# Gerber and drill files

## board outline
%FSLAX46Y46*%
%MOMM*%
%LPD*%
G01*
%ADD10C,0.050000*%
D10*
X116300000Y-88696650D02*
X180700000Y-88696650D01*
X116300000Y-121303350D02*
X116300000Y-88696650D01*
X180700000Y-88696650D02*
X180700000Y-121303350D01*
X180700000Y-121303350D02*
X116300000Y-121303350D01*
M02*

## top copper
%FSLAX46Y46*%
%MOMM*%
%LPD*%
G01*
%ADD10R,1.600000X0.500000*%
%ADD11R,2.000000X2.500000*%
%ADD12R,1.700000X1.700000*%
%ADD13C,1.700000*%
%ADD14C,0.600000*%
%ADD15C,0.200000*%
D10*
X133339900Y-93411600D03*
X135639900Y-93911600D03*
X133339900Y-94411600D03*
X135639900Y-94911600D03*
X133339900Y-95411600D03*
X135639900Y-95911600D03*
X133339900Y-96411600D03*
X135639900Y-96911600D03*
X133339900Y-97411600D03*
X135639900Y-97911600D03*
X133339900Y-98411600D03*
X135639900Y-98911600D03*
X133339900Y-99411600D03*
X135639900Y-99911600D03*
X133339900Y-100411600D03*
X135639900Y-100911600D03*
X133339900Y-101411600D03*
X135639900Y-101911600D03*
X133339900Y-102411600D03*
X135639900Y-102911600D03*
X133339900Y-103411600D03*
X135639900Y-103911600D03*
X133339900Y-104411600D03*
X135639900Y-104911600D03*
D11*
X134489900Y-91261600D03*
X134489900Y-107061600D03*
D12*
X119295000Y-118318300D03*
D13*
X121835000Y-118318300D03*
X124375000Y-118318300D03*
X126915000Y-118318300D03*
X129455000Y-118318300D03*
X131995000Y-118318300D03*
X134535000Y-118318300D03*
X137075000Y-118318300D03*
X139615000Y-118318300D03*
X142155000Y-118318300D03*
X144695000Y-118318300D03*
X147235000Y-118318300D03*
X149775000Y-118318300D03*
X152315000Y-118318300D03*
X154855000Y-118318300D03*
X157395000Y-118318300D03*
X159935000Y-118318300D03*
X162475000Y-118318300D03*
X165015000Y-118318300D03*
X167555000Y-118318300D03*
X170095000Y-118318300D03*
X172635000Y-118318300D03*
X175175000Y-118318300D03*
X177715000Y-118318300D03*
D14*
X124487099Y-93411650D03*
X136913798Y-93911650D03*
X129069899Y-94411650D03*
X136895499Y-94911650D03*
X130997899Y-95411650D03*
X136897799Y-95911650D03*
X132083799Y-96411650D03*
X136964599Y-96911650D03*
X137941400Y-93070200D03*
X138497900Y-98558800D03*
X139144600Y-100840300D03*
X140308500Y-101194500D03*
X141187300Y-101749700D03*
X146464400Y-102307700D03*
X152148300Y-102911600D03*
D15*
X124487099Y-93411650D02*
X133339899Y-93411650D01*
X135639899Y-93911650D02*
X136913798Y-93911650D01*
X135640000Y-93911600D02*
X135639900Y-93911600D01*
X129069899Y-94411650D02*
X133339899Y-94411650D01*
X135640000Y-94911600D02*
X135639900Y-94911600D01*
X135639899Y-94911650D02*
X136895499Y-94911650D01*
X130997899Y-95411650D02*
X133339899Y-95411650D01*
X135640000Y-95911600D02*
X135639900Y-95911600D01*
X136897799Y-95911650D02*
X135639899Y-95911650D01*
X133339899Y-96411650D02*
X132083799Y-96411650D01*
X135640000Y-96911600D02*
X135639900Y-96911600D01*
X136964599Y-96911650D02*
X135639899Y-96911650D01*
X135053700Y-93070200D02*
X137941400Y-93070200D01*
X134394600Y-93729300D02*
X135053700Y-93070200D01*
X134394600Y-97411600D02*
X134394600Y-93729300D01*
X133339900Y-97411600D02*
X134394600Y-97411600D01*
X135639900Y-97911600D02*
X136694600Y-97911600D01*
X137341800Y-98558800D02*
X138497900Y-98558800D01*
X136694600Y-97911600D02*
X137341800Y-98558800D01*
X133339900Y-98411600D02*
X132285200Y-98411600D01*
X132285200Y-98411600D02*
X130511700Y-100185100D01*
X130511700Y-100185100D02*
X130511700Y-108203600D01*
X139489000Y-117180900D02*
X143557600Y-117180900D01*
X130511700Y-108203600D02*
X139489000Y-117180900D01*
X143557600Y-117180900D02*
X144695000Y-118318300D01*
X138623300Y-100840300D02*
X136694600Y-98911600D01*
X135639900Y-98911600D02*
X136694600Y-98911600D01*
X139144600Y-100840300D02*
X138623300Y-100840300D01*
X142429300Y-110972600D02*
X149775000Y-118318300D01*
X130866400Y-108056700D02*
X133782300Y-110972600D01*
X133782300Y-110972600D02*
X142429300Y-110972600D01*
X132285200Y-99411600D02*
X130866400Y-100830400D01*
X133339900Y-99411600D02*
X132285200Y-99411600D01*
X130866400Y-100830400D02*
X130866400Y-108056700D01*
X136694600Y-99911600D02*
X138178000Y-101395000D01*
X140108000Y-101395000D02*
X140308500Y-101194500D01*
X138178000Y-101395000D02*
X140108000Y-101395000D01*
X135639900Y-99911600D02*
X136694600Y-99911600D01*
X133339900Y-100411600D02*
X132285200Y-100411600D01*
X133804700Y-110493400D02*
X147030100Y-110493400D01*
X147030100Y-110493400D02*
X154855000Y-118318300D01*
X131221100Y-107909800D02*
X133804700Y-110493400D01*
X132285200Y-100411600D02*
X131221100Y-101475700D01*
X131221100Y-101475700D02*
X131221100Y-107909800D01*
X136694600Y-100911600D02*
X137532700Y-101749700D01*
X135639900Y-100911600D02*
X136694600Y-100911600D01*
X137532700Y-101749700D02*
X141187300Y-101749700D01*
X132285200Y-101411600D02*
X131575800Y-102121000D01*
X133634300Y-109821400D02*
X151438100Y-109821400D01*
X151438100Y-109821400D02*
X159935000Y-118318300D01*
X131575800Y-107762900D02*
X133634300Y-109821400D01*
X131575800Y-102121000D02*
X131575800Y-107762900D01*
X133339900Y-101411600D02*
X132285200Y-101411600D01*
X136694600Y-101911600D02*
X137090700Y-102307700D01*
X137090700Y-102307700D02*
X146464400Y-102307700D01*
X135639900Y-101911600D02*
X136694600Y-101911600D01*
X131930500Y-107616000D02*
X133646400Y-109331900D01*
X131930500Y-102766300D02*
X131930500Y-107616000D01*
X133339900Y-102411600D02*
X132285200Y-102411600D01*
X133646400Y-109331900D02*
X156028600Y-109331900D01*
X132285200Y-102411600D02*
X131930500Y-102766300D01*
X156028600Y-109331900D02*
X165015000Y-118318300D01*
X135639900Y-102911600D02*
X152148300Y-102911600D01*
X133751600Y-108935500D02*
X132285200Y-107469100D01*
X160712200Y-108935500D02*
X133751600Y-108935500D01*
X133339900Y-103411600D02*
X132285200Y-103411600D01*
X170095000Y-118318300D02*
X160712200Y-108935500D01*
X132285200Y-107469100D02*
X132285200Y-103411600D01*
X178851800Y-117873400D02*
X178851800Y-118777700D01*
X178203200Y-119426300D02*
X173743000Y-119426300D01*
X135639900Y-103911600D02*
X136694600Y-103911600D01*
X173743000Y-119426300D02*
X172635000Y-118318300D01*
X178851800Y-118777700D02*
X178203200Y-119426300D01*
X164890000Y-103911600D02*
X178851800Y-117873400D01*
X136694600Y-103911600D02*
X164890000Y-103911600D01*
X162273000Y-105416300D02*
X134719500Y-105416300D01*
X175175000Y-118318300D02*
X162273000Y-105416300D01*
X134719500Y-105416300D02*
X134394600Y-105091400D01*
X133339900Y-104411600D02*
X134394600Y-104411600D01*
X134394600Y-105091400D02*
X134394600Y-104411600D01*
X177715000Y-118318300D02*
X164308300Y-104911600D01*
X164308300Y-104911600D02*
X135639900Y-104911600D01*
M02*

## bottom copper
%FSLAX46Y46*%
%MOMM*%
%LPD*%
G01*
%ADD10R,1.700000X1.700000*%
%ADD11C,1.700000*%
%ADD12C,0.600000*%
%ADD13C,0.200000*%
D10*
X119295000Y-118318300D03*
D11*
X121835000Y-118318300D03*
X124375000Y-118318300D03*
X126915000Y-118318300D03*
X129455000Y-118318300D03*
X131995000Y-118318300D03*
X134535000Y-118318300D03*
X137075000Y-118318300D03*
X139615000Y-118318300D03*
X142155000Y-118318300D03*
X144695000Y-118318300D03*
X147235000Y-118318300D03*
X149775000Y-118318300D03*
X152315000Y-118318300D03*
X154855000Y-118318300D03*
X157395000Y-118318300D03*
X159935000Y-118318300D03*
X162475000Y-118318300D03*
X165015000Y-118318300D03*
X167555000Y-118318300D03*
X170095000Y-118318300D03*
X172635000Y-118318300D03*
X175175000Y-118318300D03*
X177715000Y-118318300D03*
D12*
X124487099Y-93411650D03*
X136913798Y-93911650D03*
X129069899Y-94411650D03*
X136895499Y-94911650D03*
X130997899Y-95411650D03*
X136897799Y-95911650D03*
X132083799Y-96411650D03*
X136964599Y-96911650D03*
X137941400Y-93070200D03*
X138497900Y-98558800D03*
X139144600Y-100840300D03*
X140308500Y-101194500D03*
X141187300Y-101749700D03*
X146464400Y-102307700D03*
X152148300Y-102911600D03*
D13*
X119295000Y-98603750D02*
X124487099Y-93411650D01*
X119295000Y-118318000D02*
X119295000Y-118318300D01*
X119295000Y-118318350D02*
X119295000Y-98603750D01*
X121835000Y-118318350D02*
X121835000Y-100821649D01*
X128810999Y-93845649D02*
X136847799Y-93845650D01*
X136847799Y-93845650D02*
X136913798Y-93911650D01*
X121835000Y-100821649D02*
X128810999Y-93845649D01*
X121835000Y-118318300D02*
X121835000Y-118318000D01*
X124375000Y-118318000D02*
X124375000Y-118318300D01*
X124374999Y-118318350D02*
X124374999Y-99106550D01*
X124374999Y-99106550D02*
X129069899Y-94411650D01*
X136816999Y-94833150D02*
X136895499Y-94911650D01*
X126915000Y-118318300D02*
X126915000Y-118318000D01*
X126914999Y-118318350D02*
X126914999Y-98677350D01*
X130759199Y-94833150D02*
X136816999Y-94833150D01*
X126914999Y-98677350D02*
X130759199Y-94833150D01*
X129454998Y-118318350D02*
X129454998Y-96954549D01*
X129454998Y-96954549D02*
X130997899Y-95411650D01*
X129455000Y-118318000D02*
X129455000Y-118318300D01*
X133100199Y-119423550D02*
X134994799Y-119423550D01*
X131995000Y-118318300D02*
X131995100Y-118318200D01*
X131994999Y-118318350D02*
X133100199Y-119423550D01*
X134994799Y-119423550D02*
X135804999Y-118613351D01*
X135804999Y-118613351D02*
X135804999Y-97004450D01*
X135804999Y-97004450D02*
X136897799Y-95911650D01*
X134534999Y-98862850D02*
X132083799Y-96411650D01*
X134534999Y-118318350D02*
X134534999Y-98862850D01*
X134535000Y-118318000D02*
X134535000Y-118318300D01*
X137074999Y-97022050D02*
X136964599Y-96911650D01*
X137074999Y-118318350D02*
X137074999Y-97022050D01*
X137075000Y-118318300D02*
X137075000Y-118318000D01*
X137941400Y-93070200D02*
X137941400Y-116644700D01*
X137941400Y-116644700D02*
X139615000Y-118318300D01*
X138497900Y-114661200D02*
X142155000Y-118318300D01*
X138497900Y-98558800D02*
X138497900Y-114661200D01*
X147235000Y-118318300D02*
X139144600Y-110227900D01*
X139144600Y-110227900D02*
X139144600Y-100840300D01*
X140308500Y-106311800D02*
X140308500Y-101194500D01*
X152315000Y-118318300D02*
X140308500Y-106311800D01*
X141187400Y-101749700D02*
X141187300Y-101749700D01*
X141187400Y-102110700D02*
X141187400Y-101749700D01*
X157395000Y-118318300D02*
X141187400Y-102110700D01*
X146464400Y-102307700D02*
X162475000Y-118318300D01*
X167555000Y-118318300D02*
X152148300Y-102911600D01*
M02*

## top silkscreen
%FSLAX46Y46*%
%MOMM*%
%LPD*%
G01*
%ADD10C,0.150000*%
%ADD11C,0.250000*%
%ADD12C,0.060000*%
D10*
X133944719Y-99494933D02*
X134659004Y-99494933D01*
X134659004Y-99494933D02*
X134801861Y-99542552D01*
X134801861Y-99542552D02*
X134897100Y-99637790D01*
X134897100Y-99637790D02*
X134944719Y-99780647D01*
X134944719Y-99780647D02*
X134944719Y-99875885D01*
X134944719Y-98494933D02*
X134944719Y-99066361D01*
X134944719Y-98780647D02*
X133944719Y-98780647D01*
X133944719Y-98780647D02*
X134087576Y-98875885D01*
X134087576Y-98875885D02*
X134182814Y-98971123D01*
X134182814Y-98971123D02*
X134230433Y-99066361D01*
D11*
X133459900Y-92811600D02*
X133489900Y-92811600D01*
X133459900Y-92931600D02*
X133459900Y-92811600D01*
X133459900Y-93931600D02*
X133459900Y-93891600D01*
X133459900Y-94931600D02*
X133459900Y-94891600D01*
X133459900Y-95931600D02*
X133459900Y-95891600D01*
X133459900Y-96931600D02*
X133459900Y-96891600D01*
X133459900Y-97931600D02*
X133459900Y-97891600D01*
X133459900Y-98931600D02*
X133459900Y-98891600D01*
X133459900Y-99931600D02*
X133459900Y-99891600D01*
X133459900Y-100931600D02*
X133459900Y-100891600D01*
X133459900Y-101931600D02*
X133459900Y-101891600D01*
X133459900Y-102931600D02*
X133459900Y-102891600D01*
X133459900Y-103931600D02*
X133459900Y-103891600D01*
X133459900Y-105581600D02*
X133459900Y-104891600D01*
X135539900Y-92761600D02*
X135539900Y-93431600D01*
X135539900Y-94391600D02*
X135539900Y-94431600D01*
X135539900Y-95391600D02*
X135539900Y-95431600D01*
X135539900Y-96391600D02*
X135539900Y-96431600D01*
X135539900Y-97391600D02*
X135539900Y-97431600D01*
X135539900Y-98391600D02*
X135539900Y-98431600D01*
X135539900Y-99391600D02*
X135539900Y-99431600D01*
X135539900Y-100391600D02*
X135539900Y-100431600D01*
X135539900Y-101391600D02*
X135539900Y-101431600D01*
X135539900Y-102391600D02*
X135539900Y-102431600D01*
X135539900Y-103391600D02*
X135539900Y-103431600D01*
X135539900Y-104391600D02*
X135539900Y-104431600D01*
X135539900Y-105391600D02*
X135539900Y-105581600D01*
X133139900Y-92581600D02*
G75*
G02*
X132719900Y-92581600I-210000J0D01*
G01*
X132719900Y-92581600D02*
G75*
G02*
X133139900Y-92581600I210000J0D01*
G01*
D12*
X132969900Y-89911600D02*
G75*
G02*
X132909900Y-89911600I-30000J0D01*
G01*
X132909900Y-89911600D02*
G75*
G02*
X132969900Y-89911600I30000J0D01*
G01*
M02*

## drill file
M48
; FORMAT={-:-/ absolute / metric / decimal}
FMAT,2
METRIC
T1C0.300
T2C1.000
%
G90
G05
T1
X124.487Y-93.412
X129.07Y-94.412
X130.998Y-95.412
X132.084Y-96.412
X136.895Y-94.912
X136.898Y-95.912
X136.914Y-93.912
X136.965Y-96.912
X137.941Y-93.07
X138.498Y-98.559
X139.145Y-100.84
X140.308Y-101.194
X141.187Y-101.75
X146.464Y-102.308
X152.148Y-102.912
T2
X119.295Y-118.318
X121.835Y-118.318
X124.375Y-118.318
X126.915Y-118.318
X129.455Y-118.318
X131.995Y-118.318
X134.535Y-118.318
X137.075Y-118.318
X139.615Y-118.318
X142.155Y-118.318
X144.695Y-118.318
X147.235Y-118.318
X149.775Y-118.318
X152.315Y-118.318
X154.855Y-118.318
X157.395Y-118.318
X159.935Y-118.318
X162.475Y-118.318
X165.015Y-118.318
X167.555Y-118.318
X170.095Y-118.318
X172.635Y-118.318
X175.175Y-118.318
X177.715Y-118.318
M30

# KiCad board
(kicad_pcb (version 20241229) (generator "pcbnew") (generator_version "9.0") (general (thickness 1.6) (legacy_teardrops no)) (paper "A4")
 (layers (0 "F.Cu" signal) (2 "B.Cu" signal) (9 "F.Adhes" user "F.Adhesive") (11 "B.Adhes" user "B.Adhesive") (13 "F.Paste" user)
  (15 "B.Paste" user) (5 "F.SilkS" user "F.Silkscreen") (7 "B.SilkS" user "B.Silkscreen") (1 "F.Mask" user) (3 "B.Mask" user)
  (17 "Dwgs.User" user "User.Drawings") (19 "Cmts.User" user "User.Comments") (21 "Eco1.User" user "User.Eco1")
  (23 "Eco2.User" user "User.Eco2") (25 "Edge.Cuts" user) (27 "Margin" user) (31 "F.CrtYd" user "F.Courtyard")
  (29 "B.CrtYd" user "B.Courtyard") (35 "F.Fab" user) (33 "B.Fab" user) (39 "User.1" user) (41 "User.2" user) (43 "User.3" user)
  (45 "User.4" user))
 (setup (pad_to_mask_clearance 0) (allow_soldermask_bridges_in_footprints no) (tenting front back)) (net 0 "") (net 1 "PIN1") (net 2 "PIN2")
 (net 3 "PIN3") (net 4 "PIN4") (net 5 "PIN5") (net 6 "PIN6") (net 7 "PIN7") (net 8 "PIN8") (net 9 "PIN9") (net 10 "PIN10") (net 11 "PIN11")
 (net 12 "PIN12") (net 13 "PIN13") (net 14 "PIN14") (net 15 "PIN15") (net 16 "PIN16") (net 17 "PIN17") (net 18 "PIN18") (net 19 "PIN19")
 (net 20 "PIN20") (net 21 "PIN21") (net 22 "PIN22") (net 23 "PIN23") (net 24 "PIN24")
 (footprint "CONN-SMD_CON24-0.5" (layer "F.Cu") (at 134.4899 99.1616 -90)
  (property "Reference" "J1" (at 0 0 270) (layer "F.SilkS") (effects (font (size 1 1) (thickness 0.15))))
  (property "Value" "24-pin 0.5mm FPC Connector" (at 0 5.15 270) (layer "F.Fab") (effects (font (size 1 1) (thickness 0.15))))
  (fp_line (start -6.35 1.03) (end -6.35 1) (stroke (width 0.25) (type solid)) (layer "F.SilkS"))
  (fp_line (start -6.23 1.03) (end -6.35 1.03) (stroke (width 0.25) (type solid)) (layer "F.SilkS"))
  (fp_line (start -5.23 1.03) (end -5.27 1.03) (stroke (width 0.25) (type solid)) (layer "F.SilkS"))
  (fp_line (start -4.23 1.03) (end -4.27 1.03) (stroke (width 0.25) (type solid)) (layer "F.SilkS"))
  (fp_line (start -3.23 1.03) (end -3.27 1.03) (stroke (width 0.25) (type solid)) (layer "F.SilkS"))
  (fp_line (start -2.23 1.03) (end -2.27 1.03) (stroke (width 0.25) (type solid)) (layer "F.SilkS"))
  (fp_line (start -1.23 1.03) (end -1.27 1.03) (stroke (width 0.25) (type solid)) (layer "F.SilkS"))
  (fp_line (start -0.23 1.03) (end -0.27 1.03) (stroke (width 0.25) (type solid)) (layer "F.SilkS"))
  (fp_line (start 0.77 1.03) (end 0.73 1.03) (stroke (width 0.25) (type solid)) (layer "F.SilkS"))
  (fp_line (start 1.77 1.03) (end 1.73 1.03) (stroke (width 0.25) (type solid)) (layer "F.SilkS"))
  (fp_line (start 2.77 1.03) (end 2.73 1.03) (stroke (width 0.25) (type solid)) (layer "F.SilkS"))
  (fp_line (start 3.77 1.03) (end 3.73 1.03) (stroke (width 0.25) (type solid)) (layer "F.SilkS"))
  (fp_line (start 4.77 1.03) (end 4.73 1.03) (stroke (width 0.25) (type solid)) (layer "F.SilkS"))
  (fp_line (start 6.42 1.03) (end 5.73 1.03) (stroke (width 0.25) (type solid)) (layer "F.SilkS"))
  (fp_line (start -6.4 -1.05) (end -5.73 -1.05) (stroke (width 0.25) (type solid)) (layer "F.SilkS"))
  (fp_line (start -4.77 -1.05) (end -4.73 -1.05) (stroke (width 0.25) (type solid)) (layer "F.SilkS"))
  (fp_line (start -3.77 -1.05) (end -3.73 -1.05) (stroke (width 0.25) (type solid)) (layer "F.SilkS"))
  (fp_line (start -2.77 -1.05) (end -2.73 -1.05) (stroke (width 0.25) (type solid)) (layer "F.SilkS"))
  (fp_line (start -1.77 -1.05) (end -1.73 -1.05) (stroke (width 0.25) (type solid)) (layer "F.SilkS"))
  (fp_line (start -0.77 -1.05) (end -0.73 -1.05) (stroke (width 0.25) (type solid)) (layer "F.SilkS"))
  (fp_line (start 0.23 -1.05) (end 0.27 -1.05) (stroke (width 0.25) (type solid)) (layer "F.SilkS"))
  (fp_line (start 1.23 -1.05) (end 1.27 -1.05) (stroke (width 0.25) (type solid)) (layer "F.SilkS"))
  (fp_line (start 2.23 -1.05) (end 2.27 -1.05) (stroke (width 0.25) (type solid)) (layer "F.SilkS"))
  (fp_line (start 3.23 -1.05) (end 3.27 -1.05) (stroke (width 0.25) (type solid)) (layer "F.SilkS"))
  (fp_line (start 4.23 -1.05) (end 4.27 -1.05) (stroke (width 0.25) (type solid)) (layer "F.SilkS"))
  (fp_line (start 5.23 -1.05) (end 5.27 -1.05) (stroke (width 0.25) (type solid)) (layer "F.SilkS"))
  (fp_line (start 6.23 -1.05) (end 6.42 -1.05) (stroke (width 0.25) (type solid)) (layer "F.SilkS"))
  (fp_circle (center -6.58 1.56) (end -6.37 1.56) (stroke (width 0.25) (type solid)) (fill no) (layer "F.SilkS"))
  (fp_circle (center -9.25 1.55) (end -9.22 1.55) (stroke (width 0.06) (type solid)) (fill no) (layer "F.SilkS"))
  (pad "1" smd rect (at -5.75 1.15 270) (size 0.5 1.6) (layers "F.Cu" "F.Mask" "F.Paste") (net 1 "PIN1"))
  (pad "2" smd rect (at -5.25 -1.15 270) (size 0.5 1.6) (layers "F.Cu" "F.Mask" "F.Paste") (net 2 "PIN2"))
  (pad "3" smd rect (at -4.75 1.15 270) (size 0.5 1.6) (layers "F.Cu" "F.Mask" "F.Paste") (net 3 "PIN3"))
  (pad "4" smd rect (at -4.25 -1.15 270) (size 0.5 1.6) (layers "F.Cu" "F.Mask" "F.Paste") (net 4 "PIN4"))
  (pad "5" smd rect (at -3.75 1.15 270) (size 0.5 1.6) (layers "F.Cu" "F.Mask" "F.Paste") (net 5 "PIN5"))
  (pad "6" smd rect (at -3.25 -1.15 270) (size 0.5 1.6) (layers "F.Cu" "F.Mask" "F.Paste") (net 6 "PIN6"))
  (pad "7" smd rect (at -2.75 1.15 270) (size 0.5 1.6) (layers "F.Cu" "F.Mask" "F.Paste") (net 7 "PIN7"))
  (pad "8" smd rect (at -2.25 -1.15 270) (size 0.5 1.6) (layers "F.Cu" "F.Mask" "F.Paste") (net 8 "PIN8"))
  (pad "9" smd rect (at -1.75 1.15 270) (size 0.5 1.6) (layers "F.Cu" "F.Mask" "F.Paste") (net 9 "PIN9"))
  (pad "10" smd rect (at -1.25 -1.15 270) (size 0.5 1.6) (layers "F.Cu" "F.Mask" "F.Paste") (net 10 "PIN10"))
  (pad "11" smd rect (at -0.75 1.15 270) (size 0.5 1.6) (layers "F.Cu" "F.Mask" "F.Paste") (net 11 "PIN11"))
  (pad "12" smd rect (at -0.25 -1.15 270) (size 0.5 1.6) (layers "F.Cu" "F.Mask" "F.Paste") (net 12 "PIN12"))
  (pad "13" smd rect (at 0.25 1.15 270) (size 0.5 1.6) (layers "F.Cu" "F.Mask" "F.Paste") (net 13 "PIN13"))
  (pad "14" smd rect (at 0.75 -1.15 270) (size 0.5 1.6) (layers "F.Cu" "F.Mask" "F.Paste") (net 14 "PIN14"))
  (pad "15" smd rect (at 1.25 1.15 270) (size 0.5 1.6) (layers "F.Cu" "F.Mask" "F.Paste") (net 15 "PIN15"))
  (pad "16" smd rect (at 1.75 -1.15 270) (size 0.5 1.6) (layers "F.Cu" "F.Mask" "F.Paste") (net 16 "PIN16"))
  (pad "17" smd rect (at 2.25 1.15 270) (size 0.5 1.6) (layers "F.Cu" "F.Mask" "F.Paste") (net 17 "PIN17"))
  (pad "18" smd rect (at 2.75 -1.15 270) (size 0.5 1.6) (layers "F.Cu" "F.Mask" "F.Paste") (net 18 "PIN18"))
  (pad "19" smd rect (at 3.25 1.15 270) (size 0.5 1.6) (layers "F.Cu" "F.Mask" "F.Paste") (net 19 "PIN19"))
  (pad "20" smd rect (at 3.75 -1.15 270) (size 0.5 1.6) (layers "F.Cu" "F.Mask" "F.Paste") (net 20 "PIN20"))
  (pad "21" smd rect (at 4.25 1.15 270) (size 0.5 1.6) (layers "F.Cu" "F.Mask" "F.Paste") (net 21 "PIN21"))
  (pad "22" smd rect (at 4.75 -1.15 270) (size 0.5 1.6) (layers "F.Cu" "F.Mask" "F.Paste") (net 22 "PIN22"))
  (pad "23" smd rect (at 5.25 1.15 270) (size 0.5 1.6) (layers "F.Cu" "F.Mask" "F.Paste") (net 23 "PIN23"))
  (pad "24" smd rect (at 5.75 -1.15 270) (size 0.5 1.6) (layers "F.Cu" "F.Mask" "F.Paste") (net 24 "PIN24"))
  (pad "25" smd rect (at -7.9 0 270) (size 2.5 2) (layers "F.Cu" "F.Mask" "F.Paste"))
  (pad "26" smd rect (at 7.9 0 270) (size 2.5 2) (layers "F.Cu" "F.Mask" "F.Paste")))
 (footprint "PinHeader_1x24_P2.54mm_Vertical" (layer "B.Cu") (at 119.295 118.3183 -90)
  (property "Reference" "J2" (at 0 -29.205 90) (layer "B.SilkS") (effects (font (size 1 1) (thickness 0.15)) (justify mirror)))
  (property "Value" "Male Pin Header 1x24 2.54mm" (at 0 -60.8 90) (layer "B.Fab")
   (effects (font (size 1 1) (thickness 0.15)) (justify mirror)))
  (pad "1" thru_hole rect (at 0 0 270) (size 1.7 1.7) (drill 1) (layers "*.Cu" "*.Mask") (remove_unused_layers no) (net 1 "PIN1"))
  (pad "2" thru_hole circle (at 0 -2.54 270) (size 1.7 1.7) (drill 1) (layers "*.Cu" "*.Mask") (remove_unused_layers no) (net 2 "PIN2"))
  (pad "3" thru_hole circle (at 0 -5.08 270) (size 1.7 1.7) (drill 1) (layers "*.Cu" "*.Mask") (remove_unused_layers no) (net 3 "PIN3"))
  (pad "4" thru_hole circle (at 0 -7.62 270) (size 1.7 1.7) (drill 1) (layers "*.Cu" "*.Mask") (remove_unused_layers no) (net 4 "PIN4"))
  (pad "5" thru_hole circle (at 0 -10.16 270) (size 1.7 1.7) (drill 1) (layers "*.Cu" "*.Mask") (remove_unused_layers no) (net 5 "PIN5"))
  (pad "6" thru_hole circle (at 0 -12.7 270) (size 1.7 1.7) (drill 1) (layers "*.Cu" "*.Mask") (remove_unused_layers no) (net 6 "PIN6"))
  (pad "7" thru_hole circle (at 0 -15.24 270) (size 1.7 1.7) (drill 1) (layers "*.Cu" "*.Mask") (remove_unused_layers no) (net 7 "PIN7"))
  (pad "8" thru_hole circle (at 0 -17.78 270) (size 1.7 1.7) (drill 1) (layers "*.Cu" "*.Mask") (remove_unused_layers no) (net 8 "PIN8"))
  (pad "9" thru_hole circle (at 0 -20.32 270) (size 1.7 1.7) (drill 1) (layers "*.Cu" "*.Mask") (remove_unused_layers no) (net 9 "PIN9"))
  (pad "10" thru_hole circle (at 0 -22.86 270) (size 1.7 1.7) (drill 1) (layers "*.Cu" "*.Mask") (remove_unused_layers no) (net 10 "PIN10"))
  (pad "11" thru_hole circle (at 0 -25.4 270) (size 1.7 1.7) (drill 1) (layers "*.Cu" "*.Mask") (remove_unused_layers no) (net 11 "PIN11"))
  (pad "12" thru_hole circle (at 0 -27.94 270) (size 1.7 1.7) (drill 1) (layers "*.Cu" "*.Mask") (remove_unused_layers no) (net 12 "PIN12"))
  (pad "13" thru_hole circle (at 0 -30.48 270) (size 1.7 1.7) (drill 1) (layers "*.Cu" "*.Mask") (remove_unused_layers no) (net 13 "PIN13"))
  (pad "14" thru_hole circle (at 0 -33.02 270) (size 1.7 1.7) (drill 1) (layers "*.Cu" "*.Mask") (remove_unused_layers no) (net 14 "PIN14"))
  (pad "15" thru_hole circle (at 0 -35.56 270) (size 1.7 1.7) (drill 1) (layers "*.Cu" "*.Mask") (remove_unused_layers no) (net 15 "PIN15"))
  (pad "16" thru_hole circle (at 0 -38.1 270) (size 1.7 1.7) (drill 1) (layers "*.Cu" "*.Mask") (remove_unused_layers no) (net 16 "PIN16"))
  (pad "17" thru_hole circle (at 0 -40.64 270) (size 1.7 1.7) (drill 1) (layers "*.Cu" "*.Mask") (remove_unused_layers no) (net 17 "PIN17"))
  (pad "18" thru_hole circle (at 0 -43.18 270) (size 1.7 1.7) (drill 1) (layers "*.Cu" "*.Mask") (remove_unused_layers no) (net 18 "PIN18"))
  (pad "19" thru_hole circle (at 0 -45.72 270) (size 1.7 1.7) (drill 1) (layers "*.Cu" "*.Mask") (remove_unused_layers no) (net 19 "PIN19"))
  (pad "20" thru_hole circle (at 0 -48.26 270) (size 1.7 1.7) (drill 1) (layers "*.Cu" "*.Mask") (remove_unused_layers no) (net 20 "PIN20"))
  (pad "21" thru_hole circle (at 0 -50.8 270) (size 1.7 1.7) (drill 1) (layers "*.Cu" "*.Mask") (remove_unused_layers no) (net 21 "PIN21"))
  (pad "22" thru_hole circle (at 0 -53.34 270) (size 1.7 1.7) (drill 1) (layers "*.Cu" "*.Mask") (remove_unused_layers no) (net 22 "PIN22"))
  (pad "23" thru_hole circle (at 0 -55.88 270) (size 1.7 1.7) (drill 1) (layers "*.Cu" "*.Mask") (remove_unused_layers no) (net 23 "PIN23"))
  (pad "24" thru_hole circle (at 0 -58.42 270) (size 1.7 1.7) (drill 1) (layers "*.Cu" "*.Mask") (remove_unused_layers no) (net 24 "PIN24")))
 (gr_line (start 116.3 88.69665) (end 180.7 88.69665) (stroke (width 0.05) (type default)) (layer "Edge.Cuts"))
 (gr_line (start 116.3 121.30335) (end 116.3 88.69665) (stroke (width 0.05) (type default)) (layer "Edge.Cuts"))
 (gr_line (start 180.7 88.69665) (end 180.7 121.30335) (stroke (width 0.05) (type default)) (layer "Edge.Cuts"))
 (gr_line (start 180.7 121.30335) (end 116.3 121.30335) (stroke (width 0.05) (type default)) (layer "Edge.Cuts"))
 (segment (start 124.487099 93.41165) (end 133.339899 93.41165) (width 0.2) (layer "F.Cu") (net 1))
 (via (at 124.487099 93.41165) (size 0.6) (drill 0.3) (layers "F.Cu" "B.Cu") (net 1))
 (segment (start 119.295 98.60375) (end 124.487099 93.41165) (width 0.2) (layer "B.Cu") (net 1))
 (segment (start 119.295 118.318) (end 119.295 118.3183) (width 0.2) (layer "B.Cu") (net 1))
 (segment (start 119.295 118.31835) (end 119.295 98.60375) (width 0.2) (layer "B.Cu") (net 1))
 (segment (start 135.639899 93.91165) (end 136.913798 93.91165) (width 0.2) (layer "F.Cu") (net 2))
 (segment (start 135.64 93.9116) (end 135.6399 93.9116) (width 0.2) (layer "F.Cu") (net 2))
 (via (at 136.913798 93.91165) (size 0.6) (drill 0.3) (layers "F.Cu" "B.Cu") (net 2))
 (segment (start 121.835 118.31835) (end 121.835 100.821649) (width 0.2) (layer "B.Cu") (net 2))
 (segment (start 128.810999 93.845649) (end 136.847799 93.84565) (width 0.2) (layer "B.Cu") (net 2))
 (segment (start 136.847799 93.84565) (end 136.913798 93.91165) (width 0.2) (layer "B.Cu") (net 2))
 (segment (start 121.835 100.821649) (end 128.810999 93.845649) (width 0.2) (layer "B.Cu") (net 2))
 (segment (start 121.835 118.3183) (end 121.835 118.318) (width 0.2) (layer "B.Cu") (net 2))
 (segment (start 129.069899 94.41165) (end 133.339899 94.41165) (width 0.2) (layer "F.Cu") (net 3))
 (via (at 129.069899 94.41165) (size 0.6) (drill 0.3) (layers "F.Cu" "B.Cu") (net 3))
 (segment (start 124.375 118.318) (end 124.375 118.3183) (width 0.2) (layer "B.Cu") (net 3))
 (segment (start 124.374999 118.31835) (end 124.374999 99.10655) (width 0.2) (layer "B.Cu") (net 3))
 (segment (start 124.374999 99.10655) (end 129.069899 94.41165) (width 0.2) (layer "B.Cu") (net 3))
 (segment (start 135.64 94.9116) (end 135.6399 94.9116) (width 0.2) (layer "F.Cu") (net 4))
 (segment (start 135.639899 94.91165) (end 136.895499 94.91165) (width 0.2) (layer "F.Cu") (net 4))
 (via (at 136.895499 94.91165) (size 0.6) (drill 0.3) (layers "F.Cu" "B.Cu") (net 4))
 (segment (start 136.816999 94.83315) (end 136.895499 94.91165) (width 0.2) (layer "B.Cu") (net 4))
 (segment (start 126.915 118.3183) (end 126.915 118.318) (width 0.2) (layer "B.Cu") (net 4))
 (segment (start 126.914999 118.31835) (end 126.914999 98.67735) (width 0.2) (layer "B.Cu") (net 4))
 (segment (start 130.759199 94.83315) (end 136.816999 94.83315) (width 0.2) (layer "B.Cu") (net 4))
 (segment (start 126.914999 98.67735) (end 130.759199 94.83315) (width 0.2) (layer "B.Cu") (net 4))
 (segment (start 130.997899 95.41165) (end 133.339899 95.41165) (width 0.2) (layer "F.Cu") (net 5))
 (via (at 130.997899 95.41165) (size 0.6) (drill 0.3) (layers "F.Cu" "B.Cu") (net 5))
 (segment (start 129.454998 118.31835) (end 129.454998 96.954549) (width 0.2) (layer "B.Cu") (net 5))
 (segment (start 129.454998 96.954549) (end 130.997899 95.41165) (width 0.2) (layer "B.Cu") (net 5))
 (segment (start 129.455 118.318) (end 129.455 118.3183) (width 0.2) (layer "B.Cu") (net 5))
 (segment (start 135.64 95.9116) (end 135.6399 95.9116) (width 0.2) (layer "F.Cu") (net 6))
 (segment (start 136.897799 95.91165) (end 135.639899 95.91165) (width 0.2) (layer "F.Cu") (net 6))
 (via (at 136.897799 95.91165) (size 0.6) (drill 0.3) (layers "F.Cu" "B.Cu") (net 6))
 (segment (start 133.100199 119.42355) (end 134.994799 119.42355) (width 0.2) (layer "B.Cu") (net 6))
 (segment (start 131.995 118.3183) (end 131.9951 118.3182) (width 0.2) (layer "B.Cu") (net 6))
 (segment (start 131.994999 118.31835) (end 133.100199 119.42355) (width 0.2) (layer "B.Cu") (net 6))
 (segment (start 134.994799 119.42355) (end 135.804999 118.613351) (width 0.2) (layer "B.Cu") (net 6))
 (segment (start 135.804999 118.613351) (end 135.804999 97.00445) (width 0.2) (layer "B.Cu") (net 6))
 (segment (start 135.804999 97.00445) (end 136.897799 95.91165) (width 0.2) (layer "B.Cu") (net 6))
 (segment (start 133.339899 96.41165) (end 132.083799 96.41165) (width 0.2) (layer "F.Cu") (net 7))
 (via (at 132.083799 96.41165) (size 0.6) (drill 0.3) (layers "F.Cu" "B.Cu") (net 7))
 (segment (start 134.534999 98.86285) (end 132.083799 96.41165) (width 0.2) (layer "B.Cu") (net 7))
 (segment (start 134.534999 118.31835) (end 134.534999 98.86285) (width 0.2) (layer "B.Cu") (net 7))
 (segment (start 134.535 118.318) (end 134.535 118.3183) (width 0.2) (layer "B.Cu") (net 7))
 (segment (start 135.64 96.9116) (end 135.6399 96.9116) (width 0.2) (layer "F.Cu") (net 8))
 (segment (start 136.964599 96.91165) (end 135.639899 96.91165) (width 0.2) (layer "F.Cu") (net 8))
 (via (at 136.964599 96.91165) (size 0.6) (drill 0.3) (layers "F.Cu" "B.Cu") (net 8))
 (segment (start 137.074999 97.02205) (end 136.964599 96.91165) (width 0.2) (layer "B.Cu") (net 8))
 (segment (start 137.074999 118.31835) (end 137.074999 97.02205) (width 0.2) (layer "B.Cu") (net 8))
 (segment (start 137.075 118.3183) (end 137.075 118.318) (width 0.2) (layer "B.Cu") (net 8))
 (segment (start 135.0537 93.0702) (end 137.9414 93.0702) (width 0.2) (layer "F.Cu") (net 9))
 (segment (start 134.3946 93.7293) (end 135.0537 93.0702) (width 0.2) (layer "F.Cu") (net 9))
 (segment (start 134.3946 97.4116) (end 134.3946 93.7293) (width 0.2) (layer "F.Cu") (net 9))
 (segment (start 133.3399 97.4116) (end 134.3946 97.4116) (width 0.2) (layer "F.Cu") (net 9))
 (via (at 137.9414 93.0702) (size 0.6) (drill 0.3) (layers "F.Cu" "B.Cu") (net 9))
 (segment (start 137.9414 93.0702) (end 137.9414 116.6447) (width 0.2) (layer "B.Cu") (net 9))
 (segment (start 137.9414 116.6447) (end 139.615 118.3183) (width 0.2) (layer "B.Cu") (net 9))
 (segment (start 135.6399 97.9116) (end 136.6946 97.9116) (width 0.2) (layer "F.Cu") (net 10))
 (segment (start 137.3418 98.5588) (end 138.4979 98.5588) (width 0.2) (layer "F.Cu") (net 10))
 (segment (start 136.6946 97.9116) (end 137.3418 98.5588) (width 0.2) (layer "F.Cu") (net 10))
 (via (at 138.4979 98.5588) (size 0.6) (drill 0.3) (layers "F.Cu" "B.Cu") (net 10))
 (segment (start 138.4979 114.6612) (end 142.155 118.3183) (width 0.2) (layer "B.Cu") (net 10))
 (segment (start 138.4979 98.5588) (end 138.4979 114.6612) (width 0.2) (layer "B.Cu") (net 10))
 (segment (start 133.3399 98.4116) (end 132.2852 98.4116) (width 0.2) (layer "F.Cu") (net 11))
 (segment (start 132.2852 98.4116) (end 130.5117 100.1851) (width 0.2) (layer "F.Cu") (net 11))
 (segment (start 130.5117 100.1851) (end 130.5117 108.2036) (width 0.2) (layer "F.Cu") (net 11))
 (segment (start 139.489 117.1809) (end 143.5576 117.1809) (width 0.2) (layer "F.Cu") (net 11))
 (segment (start 130.5117 108.2036) (end 139.489 117.1809) (width 0.2) (layer "F.Cu") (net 11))
 (segment (start 143.5576 117.1809) (end 144.695 118.3183) (width 0.2) (layer "F.Cu") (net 11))
 (segment (start 138.6233 100.8403) (end 136.6946 98.9116) (width 0.2) (layer "F.Cu") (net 12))
 (segment (start 135.6399 98.9116) (end 136.6946 98.9116) (width 0.2) (layer "F.Cu") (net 12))
 (segment (start 139.1446 100.8403) (end 138.6233 100.8403) (width 0.2) (layer "F.Cu") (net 12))
 (via (at 139.1446 100.8403) (size 0.6) (drill 0.3) (layers "F.Cu" "B.Cu") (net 12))
 (segment (start 147.235 118.3183) (end 139.1446 110.2279) (width 0.2) (layer "B.Cu") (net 12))
 (segment (start 139.1446 110.2279) (end 139.1446 100.8403) (width 0.2) (layer "B.Cu") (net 12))
 (segment (start 142.4293 110.9726) (end 149.775 118.3183) (width 0.2) (layer "F.Cu") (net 13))
 (segment (start 130.8664 108.0567) (end 133.7823 110.9726) (width 0.2) (layer "F.Cu") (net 13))
 (segment (start 133.7823 110.9726) (end 142.4293 110.9726) (width 0.2) (layer "F.Cu") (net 13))
 (segment (start 132.2852 99.4116) (end 130.8664 100.8304) (width 0.2) (layer "F.Cu") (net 13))
 (segment (start 133.3399 99.4116) (end 132.2852 99.4116) (width 0.2) (layer "F.Cu") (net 13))
 (segment (start 130.8664 100.8304) (end 130.8664 108.0567) (width 0.2) (layer "F.Cu") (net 13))
 (segment (start 136.6946 99.9116) (end 138.178 101.395) (width 0.2) (layer "F.Cu") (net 14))
 (segment (start 140.108 101.395) (end 140.3085 101.1945) (width 0.2) (layer "F.Cu") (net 14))
 (segment (start 138.178 101.395) (end 140.108 101.395) (width 0.2) (layer "F.Cu") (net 14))
 (segment (start 135.6399 99.9116) (end 136.6946 99.9116) (width 0.2) (layer "F.Cu") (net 14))
 (via (at 140.3085 101.1945) (size 0.6) (drill 0.3) (layers "F.Cu" "B.Cu") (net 14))
 (segment (start 140.3085 106.3118) (end 140.3085 101.1945) (width 0.2) (layer "B.Cu") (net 14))
 (segment (start 152.315 118.3183) (end 140.3085 106.3118) (width 0.2) (layer "B.Cu") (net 14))
 (segment (start 133.3399 100.4116) (end 132.2852 100.4116) (width 0.2) (layer "F.Cu") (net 15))
 (segment (start 133.8047 110.4934) (end 147.0301 110.4934) (width 0.2) (layer "F.Cu") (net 15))
 (segment (start 147.0301 110.4934) (end 154.855 118.3183) (width 0.2) (layer "F.Cu") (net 15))
 (segment (start 131.2211 107.9098) (end 133.8047 110.4934) (width 0.2) (layer "F.Cu") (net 15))
 (segment (start 132.2852 100.4116) (end 131.2211 101.4757) (width 0.2) (layer "F.Cu") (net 15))
 (segment (start 131.2211 101.4757) (end 131.2211 107.9098) (width 0.2) (layer "F.Cu") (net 15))
 (segment (start 136.6946 100.9116) (end 137.5327 101.7497) (width 0.2) (layer "F.Cu") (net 16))
 (segment (start 135.6399 100.9116) (end 136.6946 100.9116) (width 0.2) (layer "F.Cu") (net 16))
 (segment (start 137.5327 101.7497) (end 141.1873 101.7497) (width 0.2) (layer "F.Cu") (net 16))
 (via (at 141.1873 101.7497) (size 0.6) (drill 0.3) (layers "F.Cu" "B.Cu") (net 16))
 (segment (start 141.1874 101.7497) (end 141.1873 101.7497) (width 0.2) (layer "B.Cu") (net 16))
 (segment (start 141.1874 102.1107) (end 141.1874 101.7497) (width 0.2) (layer "B.Cu") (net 16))
 (segment (start 157.395 118.3183) (end 141.1874 102.1107) (width 0.2) (layer "B.Cu") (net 16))
 (segment (start 132.2852 101.4116) (end 131.5758 102.121) (width 0.2) (layer "F.Cu") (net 17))
 (segment (start 133.6343 109.8214) (end 151.4381 109.8214) (width 0.2) (layer "F.Cu") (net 17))
 (segment (start 151.4381 109.8214) (end 159.935 118.3183) (width 0.2) (layer "F.Cu") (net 17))
 (segment (start 131.5758 107.7629) (end 133.6343 109.8214) (width 0.2) (layer "F.Cu") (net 17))
 (segment (start 131.5758 102.121) (end 131.5758 107.7629) (width 0.2) (layer "F.Cu") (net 17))
 (segment (start 133.3399 101.4116) (end 132.2852 101.4116) (width 0.2) (layer "F.Cu") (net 17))
 (segment (start 136.6946 101.9116) (end 137.0907 102.3077) (width 0.2) (layer "F.Cu") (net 18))
 (segment (start 137.0907 102.3077) (end 146.4644 102.3077) (width 0.2) (layer "F.Cu") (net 18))
 (segment (start 135.6399 101.9116) (end 136.6946 101.9116) (width 0.2) (layer "F.Cu") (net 18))
 (via (at 146.4644 102.3077) (size 0.6) (drill 0.3) (layers "F.Cu" "B.Cu") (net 18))
 (segment (start 146.4644 102.3077) (end 162.475 118.3183) (width 0.2) (layer "B.Cu") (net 18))
 (segment (start 131.9305 107.616) (end 133.6464 109.3319) (width 0.2) (layer "F.Cu") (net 19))
 (segment (start 131.9305 102.7663) (end 131.9305 107.616) (width 0.2) (layer "F.Cu") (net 19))
 (segment (start 133.3399 102.4116) (end 132.2852 102.4116) (width 0.2) (layer "F.Cu") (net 19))
 (segment (start 133.6464 109.3319) (end 156.0286 109.3319) (width 0.2) (layer "F.Cu") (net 19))
 (segment (start 132.2852 102.4116) (end 131.9305 102.7663) (width 0.2) (layer "F.Cu") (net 19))
 (segment (start 156.0286 109.3319) (end 165.015 118.3183) (width 0.2) (layer "F.Cu") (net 19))
 (segment (start 135.6399 102.9116) (end 152.1483 102.9116) (width 0.2) (layer "F.Cu") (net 20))
 (via (at 152.1483 102.9116) (size 0.6) (drill 0.3) (layers "F.Cu" "B.Cu") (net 20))
 (segment (start 167.555 118.3183) (end 152.1483 102.9116) (width 0.2) (layer "B.Cu") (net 20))
 (segment (start 133.7516 108.9355) (end 132.2852 107.4691) (width 0.2) (layer "F.Cu") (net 21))
 (segment (start 160.7122 108.9355) (end 133.7516 108.9355) (width 0.2) (layer "F.Cu") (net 21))
 (segment (start 133.3399 103.4116) (end 132.2852 103.4116) (width 0.2) (layer "F.Cu") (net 21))
 (segment (start 170.095 118.3183) (end 160.7122 108.9355) (width 0.2) (layer "F.Cu") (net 21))
 (segment (start 132.2852 107.4691) (end 132.2852 103.4116) (width 0.2) (layer "F.Cu") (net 21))
 (segment (start 178.8518 117.8734) (end 178.8518 118.7777) (width 0.2) (layer "F.Cu") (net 22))
 (segment (start 178.2032 119.4263) (end 173.743 119.4263) (width 0.2) (layer "F.Cu") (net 22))
 (segment (start 135.6399 103.9116) (end 136.6946 103.9116) (width 0.2) (layer "F.Cu") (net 22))
 (segment (start 173.743 119.4263) (end 172.635 118.3183) (width 0.2) (layer "F.Cu") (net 22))
 (segment (start 178.8518 118.7777) (end 178.2032 119.4263) (width 0.2) (layer "F.Cu") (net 22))
 (segment (start 164.89 103.9116) (end 178.8518 117.8734) (width 0.2) (layer "F.Cu") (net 22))
 (segment (start 136.6946 103.9116) (end 164.89 103.9116) (width 0.2) (layer "F.Cu") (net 22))
 (segment (start 162.273 105.4163) (end 134.7195 105.4163) (width 0.2) (layer "F.Cu") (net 23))
 (segment (start 175.175 118.3183) (end 162.273 105.4163) (width 0.2) (layer "F.Cu") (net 23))
 (segment (start 134.7195 105.4163) (end 134.3946 105.0914) (width 0.2) (layer "F.Cu") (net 23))
 (segment (start 133.3399 104.4116) (end 134.3946 104.4116) (width 0.2) (layer "F.Cu") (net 23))
 (segment (start 134.3946 105.0914) (end 134.3946 104.4116) (width 0.2) (layer "F.Cu") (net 23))
 (segment (start 177.715 118.3183) (end 164.3083 104.9116) (width 0.2) (layer "F.Cu") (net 24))
 (segment (start 164.3083 104.9116) (end 135.6399 104.9116) (width 0.2) (layer "F.Cu") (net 24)))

